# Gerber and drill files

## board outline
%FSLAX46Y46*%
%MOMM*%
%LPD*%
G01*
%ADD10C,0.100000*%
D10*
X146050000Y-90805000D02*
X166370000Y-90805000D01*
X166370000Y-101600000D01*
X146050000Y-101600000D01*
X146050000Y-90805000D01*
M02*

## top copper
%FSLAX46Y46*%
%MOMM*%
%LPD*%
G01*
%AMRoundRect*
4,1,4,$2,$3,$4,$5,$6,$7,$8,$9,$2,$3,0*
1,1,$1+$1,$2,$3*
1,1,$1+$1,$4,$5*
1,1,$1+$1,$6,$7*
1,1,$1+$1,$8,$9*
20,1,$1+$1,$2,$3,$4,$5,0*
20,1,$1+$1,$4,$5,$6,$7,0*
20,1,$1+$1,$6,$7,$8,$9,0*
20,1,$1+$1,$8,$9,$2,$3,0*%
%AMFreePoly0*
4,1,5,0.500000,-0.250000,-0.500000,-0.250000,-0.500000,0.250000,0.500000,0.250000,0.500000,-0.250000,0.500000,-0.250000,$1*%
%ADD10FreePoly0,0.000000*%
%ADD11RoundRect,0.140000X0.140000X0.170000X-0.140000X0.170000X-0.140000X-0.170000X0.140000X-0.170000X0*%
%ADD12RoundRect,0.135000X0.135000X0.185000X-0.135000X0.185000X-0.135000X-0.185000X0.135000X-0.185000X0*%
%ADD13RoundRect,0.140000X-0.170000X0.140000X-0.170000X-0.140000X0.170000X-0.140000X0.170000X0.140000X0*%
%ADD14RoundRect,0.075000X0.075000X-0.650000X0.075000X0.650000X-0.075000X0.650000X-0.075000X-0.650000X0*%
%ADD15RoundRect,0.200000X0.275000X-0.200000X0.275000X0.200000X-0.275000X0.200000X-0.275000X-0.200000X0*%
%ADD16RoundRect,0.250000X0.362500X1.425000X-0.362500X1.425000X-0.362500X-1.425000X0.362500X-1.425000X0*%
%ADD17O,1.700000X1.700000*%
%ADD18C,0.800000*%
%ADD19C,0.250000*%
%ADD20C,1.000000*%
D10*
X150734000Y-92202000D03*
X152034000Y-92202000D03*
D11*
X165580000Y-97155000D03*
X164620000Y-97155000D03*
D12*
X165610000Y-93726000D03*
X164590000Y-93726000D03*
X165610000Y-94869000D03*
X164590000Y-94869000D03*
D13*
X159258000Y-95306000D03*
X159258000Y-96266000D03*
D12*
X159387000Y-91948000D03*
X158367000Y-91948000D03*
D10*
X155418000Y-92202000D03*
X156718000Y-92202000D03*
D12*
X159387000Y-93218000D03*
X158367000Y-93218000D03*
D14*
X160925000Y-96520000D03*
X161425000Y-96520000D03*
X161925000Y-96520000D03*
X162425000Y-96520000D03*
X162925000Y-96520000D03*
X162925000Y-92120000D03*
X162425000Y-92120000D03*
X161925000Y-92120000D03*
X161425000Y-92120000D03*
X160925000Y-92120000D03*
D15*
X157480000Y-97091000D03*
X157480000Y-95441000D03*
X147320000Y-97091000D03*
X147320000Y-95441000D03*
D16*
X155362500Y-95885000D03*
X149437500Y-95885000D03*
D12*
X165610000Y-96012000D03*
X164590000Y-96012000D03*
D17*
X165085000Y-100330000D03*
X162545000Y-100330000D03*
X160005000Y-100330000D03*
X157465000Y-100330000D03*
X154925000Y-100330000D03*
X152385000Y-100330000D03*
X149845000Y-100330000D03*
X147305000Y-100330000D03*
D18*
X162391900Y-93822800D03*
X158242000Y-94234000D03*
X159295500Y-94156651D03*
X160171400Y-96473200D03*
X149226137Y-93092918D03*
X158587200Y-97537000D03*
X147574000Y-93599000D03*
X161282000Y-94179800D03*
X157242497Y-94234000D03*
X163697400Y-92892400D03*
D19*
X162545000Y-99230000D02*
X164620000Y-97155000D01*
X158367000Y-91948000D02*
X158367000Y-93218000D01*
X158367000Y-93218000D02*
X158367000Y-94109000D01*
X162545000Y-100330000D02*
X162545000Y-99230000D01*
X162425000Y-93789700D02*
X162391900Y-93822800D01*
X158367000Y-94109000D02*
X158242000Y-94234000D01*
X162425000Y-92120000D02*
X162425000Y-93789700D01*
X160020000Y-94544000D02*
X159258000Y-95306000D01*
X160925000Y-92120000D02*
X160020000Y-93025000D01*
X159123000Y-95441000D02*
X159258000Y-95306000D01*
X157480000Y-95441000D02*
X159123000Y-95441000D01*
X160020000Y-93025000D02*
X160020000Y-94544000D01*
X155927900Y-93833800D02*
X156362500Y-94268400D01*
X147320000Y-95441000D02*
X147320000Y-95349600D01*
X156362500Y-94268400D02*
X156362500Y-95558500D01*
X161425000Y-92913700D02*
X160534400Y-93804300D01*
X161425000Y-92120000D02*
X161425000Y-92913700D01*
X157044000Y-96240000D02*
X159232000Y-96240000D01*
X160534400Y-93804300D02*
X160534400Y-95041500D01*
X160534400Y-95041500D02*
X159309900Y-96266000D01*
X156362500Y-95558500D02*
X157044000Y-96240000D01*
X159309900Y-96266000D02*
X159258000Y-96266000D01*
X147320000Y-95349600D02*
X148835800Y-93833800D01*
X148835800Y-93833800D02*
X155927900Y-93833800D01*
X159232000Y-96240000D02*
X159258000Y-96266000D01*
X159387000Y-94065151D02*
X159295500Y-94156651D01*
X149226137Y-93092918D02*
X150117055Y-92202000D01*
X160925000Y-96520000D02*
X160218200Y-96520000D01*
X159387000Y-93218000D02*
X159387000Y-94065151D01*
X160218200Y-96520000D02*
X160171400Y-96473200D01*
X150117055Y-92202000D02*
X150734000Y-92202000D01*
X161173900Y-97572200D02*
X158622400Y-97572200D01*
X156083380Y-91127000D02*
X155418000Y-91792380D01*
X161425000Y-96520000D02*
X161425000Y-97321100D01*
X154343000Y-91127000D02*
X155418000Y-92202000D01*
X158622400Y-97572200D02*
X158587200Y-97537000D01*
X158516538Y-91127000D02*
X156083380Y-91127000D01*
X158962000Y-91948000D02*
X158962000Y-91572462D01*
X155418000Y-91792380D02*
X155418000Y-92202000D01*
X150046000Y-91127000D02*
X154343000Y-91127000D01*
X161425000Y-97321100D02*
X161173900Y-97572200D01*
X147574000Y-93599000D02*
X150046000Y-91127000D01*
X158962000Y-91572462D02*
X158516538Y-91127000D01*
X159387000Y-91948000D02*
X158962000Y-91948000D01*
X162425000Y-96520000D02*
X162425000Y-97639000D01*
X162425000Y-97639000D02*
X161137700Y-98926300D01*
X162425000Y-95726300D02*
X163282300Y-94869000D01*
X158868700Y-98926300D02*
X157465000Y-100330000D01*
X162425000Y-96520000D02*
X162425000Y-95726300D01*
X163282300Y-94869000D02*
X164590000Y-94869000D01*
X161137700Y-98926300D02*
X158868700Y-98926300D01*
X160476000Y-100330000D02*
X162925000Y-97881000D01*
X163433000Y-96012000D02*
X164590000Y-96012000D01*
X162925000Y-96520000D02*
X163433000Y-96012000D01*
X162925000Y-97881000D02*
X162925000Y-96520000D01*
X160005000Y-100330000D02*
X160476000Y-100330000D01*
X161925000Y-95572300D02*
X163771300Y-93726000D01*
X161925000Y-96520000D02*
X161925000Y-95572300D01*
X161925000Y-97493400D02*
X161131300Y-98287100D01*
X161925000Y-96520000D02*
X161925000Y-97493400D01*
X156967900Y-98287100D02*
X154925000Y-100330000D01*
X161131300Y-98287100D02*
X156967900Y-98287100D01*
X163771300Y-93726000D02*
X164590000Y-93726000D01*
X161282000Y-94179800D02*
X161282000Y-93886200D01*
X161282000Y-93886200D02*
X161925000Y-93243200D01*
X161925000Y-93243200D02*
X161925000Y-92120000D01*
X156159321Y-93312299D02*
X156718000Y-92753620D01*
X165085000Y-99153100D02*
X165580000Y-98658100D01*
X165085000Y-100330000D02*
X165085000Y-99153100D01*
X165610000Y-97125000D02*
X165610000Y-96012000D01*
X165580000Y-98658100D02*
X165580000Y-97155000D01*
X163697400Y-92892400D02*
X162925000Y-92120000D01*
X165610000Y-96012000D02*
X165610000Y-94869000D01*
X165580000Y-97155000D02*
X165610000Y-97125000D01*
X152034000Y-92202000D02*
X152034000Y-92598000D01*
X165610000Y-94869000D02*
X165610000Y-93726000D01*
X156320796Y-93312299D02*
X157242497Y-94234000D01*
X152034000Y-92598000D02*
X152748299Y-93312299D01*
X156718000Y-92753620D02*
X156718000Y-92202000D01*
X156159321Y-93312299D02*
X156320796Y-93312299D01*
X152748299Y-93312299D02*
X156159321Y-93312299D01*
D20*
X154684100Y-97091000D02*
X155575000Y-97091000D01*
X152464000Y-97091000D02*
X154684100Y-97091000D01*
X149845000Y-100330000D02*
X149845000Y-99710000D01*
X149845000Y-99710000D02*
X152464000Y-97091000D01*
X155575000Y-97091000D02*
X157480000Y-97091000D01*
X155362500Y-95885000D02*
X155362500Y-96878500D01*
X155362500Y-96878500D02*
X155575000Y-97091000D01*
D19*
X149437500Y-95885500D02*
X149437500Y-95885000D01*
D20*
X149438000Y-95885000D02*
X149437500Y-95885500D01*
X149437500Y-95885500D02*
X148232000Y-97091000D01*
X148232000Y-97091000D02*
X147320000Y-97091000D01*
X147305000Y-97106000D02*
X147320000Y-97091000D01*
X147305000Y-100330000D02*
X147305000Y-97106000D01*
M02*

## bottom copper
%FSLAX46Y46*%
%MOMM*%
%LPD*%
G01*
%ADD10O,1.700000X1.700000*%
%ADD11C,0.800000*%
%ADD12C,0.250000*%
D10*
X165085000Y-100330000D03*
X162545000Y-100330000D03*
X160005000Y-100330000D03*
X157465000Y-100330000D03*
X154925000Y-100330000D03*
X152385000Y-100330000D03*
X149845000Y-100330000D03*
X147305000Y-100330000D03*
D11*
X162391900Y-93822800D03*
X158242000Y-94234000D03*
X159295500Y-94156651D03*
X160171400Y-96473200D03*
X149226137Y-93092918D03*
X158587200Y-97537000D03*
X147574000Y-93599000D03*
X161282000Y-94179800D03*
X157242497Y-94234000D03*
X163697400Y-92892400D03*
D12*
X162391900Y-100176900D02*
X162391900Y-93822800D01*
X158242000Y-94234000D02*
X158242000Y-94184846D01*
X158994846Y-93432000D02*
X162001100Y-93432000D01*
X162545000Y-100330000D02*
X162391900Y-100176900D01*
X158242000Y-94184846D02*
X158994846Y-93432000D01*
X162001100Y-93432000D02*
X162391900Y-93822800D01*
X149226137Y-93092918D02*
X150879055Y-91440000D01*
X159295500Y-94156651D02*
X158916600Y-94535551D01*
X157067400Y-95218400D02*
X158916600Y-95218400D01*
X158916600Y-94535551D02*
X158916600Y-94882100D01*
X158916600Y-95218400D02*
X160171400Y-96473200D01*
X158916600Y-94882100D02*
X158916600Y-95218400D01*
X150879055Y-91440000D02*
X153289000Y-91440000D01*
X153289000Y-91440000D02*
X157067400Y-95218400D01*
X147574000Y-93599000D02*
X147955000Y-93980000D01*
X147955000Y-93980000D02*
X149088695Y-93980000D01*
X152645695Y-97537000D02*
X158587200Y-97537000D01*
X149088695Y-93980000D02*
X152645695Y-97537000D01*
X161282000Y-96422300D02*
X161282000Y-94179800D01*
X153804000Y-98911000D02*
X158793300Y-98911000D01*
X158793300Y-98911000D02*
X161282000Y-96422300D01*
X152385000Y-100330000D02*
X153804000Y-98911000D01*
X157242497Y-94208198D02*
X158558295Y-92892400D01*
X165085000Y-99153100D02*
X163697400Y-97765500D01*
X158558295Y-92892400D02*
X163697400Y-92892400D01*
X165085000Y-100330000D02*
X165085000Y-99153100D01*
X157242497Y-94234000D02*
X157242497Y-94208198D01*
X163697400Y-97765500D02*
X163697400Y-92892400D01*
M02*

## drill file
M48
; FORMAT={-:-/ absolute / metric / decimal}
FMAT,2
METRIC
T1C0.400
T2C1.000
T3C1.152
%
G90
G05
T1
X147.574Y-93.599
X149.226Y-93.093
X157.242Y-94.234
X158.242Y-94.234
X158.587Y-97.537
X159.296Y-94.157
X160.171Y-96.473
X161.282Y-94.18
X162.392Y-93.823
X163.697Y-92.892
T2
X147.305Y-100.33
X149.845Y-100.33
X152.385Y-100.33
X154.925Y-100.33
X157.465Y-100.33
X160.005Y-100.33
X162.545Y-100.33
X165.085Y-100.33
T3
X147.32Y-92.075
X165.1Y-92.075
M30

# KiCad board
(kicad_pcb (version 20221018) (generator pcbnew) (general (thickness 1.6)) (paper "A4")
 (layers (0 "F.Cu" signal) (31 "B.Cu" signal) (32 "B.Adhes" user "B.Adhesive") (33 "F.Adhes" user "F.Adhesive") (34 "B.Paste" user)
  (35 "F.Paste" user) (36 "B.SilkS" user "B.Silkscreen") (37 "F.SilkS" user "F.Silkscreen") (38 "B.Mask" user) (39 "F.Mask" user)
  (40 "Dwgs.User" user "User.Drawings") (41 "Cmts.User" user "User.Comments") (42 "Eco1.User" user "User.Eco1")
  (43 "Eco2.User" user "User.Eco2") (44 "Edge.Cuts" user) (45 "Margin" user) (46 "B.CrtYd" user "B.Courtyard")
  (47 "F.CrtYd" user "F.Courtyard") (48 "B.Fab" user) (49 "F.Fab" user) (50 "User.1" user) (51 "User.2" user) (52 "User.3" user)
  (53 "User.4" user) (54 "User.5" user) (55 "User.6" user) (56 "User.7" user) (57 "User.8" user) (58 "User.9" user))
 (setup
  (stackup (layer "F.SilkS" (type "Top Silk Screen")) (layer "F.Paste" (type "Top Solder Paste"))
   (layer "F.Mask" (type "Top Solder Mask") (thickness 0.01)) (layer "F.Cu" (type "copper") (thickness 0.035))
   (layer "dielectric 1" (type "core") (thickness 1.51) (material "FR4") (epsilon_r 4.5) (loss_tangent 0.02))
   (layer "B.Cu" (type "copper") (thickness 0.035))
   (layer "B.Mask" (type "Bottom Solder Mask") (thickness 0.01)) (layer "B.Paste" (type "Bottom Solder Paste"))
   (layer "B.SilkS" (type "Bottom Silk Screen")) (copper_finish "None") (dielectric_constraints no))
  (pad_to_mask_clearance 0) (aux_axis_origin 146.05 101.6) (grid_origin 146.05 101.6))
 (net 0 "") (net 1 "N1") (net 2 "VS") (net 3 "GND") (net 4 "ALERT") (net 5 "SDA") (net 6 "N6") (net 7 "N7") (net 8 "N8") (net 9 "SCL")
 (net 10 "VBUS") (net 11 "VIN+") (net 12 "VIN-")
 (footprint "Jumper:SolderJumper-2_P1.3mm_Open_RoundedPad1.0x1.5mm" (layer "F.Cu") (at 151.384 92.202)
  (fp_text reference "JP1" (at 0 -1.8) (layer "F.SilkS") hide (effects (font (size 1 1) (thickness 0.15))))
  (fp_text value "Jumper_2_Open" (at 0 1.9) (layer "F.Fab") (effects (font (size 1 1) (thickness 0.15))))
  (pad "1" smd custom (at -0.65 0) (size 1 0.5) (layers "F.Cu" "F.Mask") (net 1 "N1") (zone_connect 2) (thermal_bridge_angle 45)
   (options (clearance outline) (anchor rect)) (primitives))
  (pad "2" smd custom (at 0.65 0) (size 1 0.5) (layers "F.Cu" "F.Mask") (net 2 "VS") (zone_connect 2) (thermal_bridge_angle 45)
   (options (clearance outline) (anchor rect)) (primitives)))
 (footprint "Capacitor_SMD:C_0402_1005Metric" (layer "F.Cu") (at 165.1 97.155 180)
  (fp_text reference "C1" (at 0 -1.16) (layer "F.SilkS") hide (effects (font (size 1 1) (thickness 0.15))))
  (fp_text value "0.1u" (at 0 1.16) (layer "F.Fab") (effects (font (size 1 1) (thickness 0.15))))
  (pad "1" smd roundrect (at -0.48 0 180) (size 0.56 0.62) (layers "F.Cu" "F.Paste" "F.Mask") (roundrect_rratio 0.25) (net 2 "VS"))
  (pad "2" smd roundrect (at 0.48 0 180) (size 0.56 0.62) (layers "F.Cu" "F.Paste" "F.Mask") (roundrect_rratio 0.25) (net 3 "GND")))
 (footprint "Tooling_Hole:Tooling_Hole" (layer "F.Cu") (at 165.1 92.075)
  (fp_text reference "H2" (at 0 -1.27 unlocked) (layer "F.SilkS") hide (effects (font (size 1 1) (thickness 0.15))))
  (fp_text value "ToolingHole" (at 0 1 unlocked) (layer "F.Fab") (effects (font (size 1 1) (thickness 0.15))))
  (pad "" np_thru_hole circle (at 0 0) (size 1.152 1.152) (drill 1.152) (layers "F&B.Cu" "*.Mask")))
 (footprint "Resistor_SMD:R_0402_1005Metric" (layer "F.Cu") (at 165.1 93.726 180)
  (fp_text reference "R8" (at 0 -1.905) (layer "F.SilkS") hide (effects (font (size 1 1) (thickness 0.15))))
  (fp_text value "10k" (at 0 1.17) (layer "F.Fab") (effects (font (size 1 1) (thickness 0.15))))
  (pad "1" smd roundrect (at -0.51 0 180) (size 0.54 0.64) (layers "F.Cu" "F.Paste" "F.Mask") (roundrect_rratio 0.25) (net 2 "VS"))
  (pad "2" smd roundrect (at 0.51 0 180) (size 0.54 0.64) (layers "F.Cu" "F.Paste" "F.Mask") (roundrect_rratio 0.25) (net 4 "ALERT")))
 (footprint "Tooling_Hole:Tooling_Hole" (layer "F.Cu") (at 147.32 92.075)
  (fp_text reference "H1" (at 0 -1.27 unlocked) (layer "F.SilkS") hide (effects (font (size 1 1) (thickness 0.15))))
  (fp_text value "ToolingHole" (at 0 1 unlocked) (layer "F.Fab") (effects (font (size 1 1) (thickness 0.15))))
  (pad "" np_thru_hole circle (at 0 0) (size 1.152 1.152) (drill 1.152) (layers "F&B.Cu" "*.Mask")))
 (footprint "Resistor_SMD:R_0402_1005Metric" (layer "F.Cu") (at 165.1 94.869 180)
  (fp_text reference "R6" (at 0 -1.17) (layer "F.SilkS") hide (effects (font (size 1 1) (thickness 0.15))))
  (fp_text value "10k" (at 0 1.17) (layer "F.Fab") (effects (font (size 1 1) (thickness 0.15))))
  (pad "1" smd roundrect (at -0.51 0 180) (size 0.54 0.64) (layers "F.Cu" "F.Paste" "F.Mask") (roundrect_rratio 0.25) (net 2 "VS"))
  (pad "2" smd roundrect (at 0.51 0 180) (size 0.54 0.64) (layers "F.Cu" "F.Paste" "F.Mask") (roundrect_rratio 0.25) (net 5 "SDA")))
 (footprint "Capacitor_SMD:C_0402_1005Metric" (layer "F.Cu") (at 159.258 95.786 -90)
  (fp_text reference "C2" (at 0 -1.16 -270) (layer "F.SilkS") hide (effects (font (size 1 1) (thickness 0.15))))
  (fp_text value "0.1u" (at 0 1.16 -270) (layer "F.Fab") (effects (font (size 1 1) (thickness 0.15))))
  (pad "1" smd roundrect (at -0.48 0 270) (size 0.56 0.62) (layers "F.Cu" "F.Paste" "F.Mask") (roundrect_rratio 0.25) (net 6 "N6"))
  (pad "2" smd roundrect (at 0.48 0 270) (size 0.56 0.62) (layers "F.Cu" "F.Paste" "F.Mask") (roundrect_rratio 0.25) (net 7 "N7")))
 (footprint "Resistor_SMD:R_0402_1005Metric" (layer "F.Cu") (at 158.877 91.948 180)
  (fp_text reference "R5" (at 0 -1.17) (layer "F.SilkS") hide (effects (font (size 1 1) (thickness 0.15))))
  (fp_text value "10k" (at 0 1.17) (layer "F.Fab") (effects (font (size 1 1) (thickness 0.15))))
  (pad "1" smd roundrect (at -0.51 0 180) (size 0.54 0.64) (layers "F.Cu" "F.Paste" "F.Mask") (roundrect_rratio 0.25) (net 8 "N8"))
  (pad "2" smd roundrect (at 0.51 0 180) (size 0.54 0.64) (layers "F.Cu" "F.Paste" "F.Mask") (roundrect_rratio 0.25) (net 3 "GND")))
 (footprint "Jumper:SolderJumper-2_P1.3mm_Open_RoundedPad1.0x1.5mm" (layer "F.Cu") (at 156.068 92.202)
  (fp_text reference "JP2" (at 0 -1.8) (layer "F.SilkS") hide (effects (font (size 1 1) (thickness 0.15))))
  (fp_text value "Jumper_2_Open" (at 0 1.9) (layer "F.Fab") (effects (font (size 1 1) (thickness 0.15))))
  (pad "1" smd custom (at -0.65 0) (size 1 0.5) (layers "F.Cu" "F.Mask") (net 8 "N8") (zone_connect 2) (thermal_bridge_angle 45)
   (options (clearance outline) (anchor rect)) (primitives))
  (pad "2" smd custom (at 0.65 0) (size 1 0.5) (layers "F.Cu" "F.Mask") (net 2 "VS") (zone_connect 2) (thermal_bridge_angle 45)
   (options (clearance outline) (anchor rect)) (primitives)))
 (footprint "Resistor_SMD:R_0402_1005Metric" (layer "F.Cu") (at 158.877 93.218 180)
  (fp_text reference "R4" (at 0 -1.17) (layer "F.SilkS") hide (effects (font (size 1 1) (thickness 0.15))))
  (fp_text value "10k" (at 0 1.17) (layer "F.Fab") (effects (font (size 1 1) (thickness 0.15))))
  (pad "1" smd roundrect (at -0.51 0 180) (size 0.54 0.64) (layers "F.Cu" "F.Paste" "F.Mask") (roundrect_rratio 0.25) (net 1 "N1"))
  (pad "2" smd roundrect (at 0.51 0 180) (size 0.54 0.64) (layers "F.Cu" "F.Paste" "F.Mask") (roundrect_rratio 0.25) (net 3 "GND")))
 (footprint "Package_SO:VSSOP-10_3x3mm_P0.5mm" (layer "F.Cu") (at 161.925 94.32 90)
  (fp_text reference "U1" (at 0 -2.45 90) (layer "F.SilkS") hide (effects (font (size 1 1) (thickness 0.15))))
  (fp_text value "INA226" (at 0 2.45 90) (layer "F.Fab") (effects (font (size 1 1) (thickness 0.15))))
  (pad "1" smd roundrect (at -2.2 -1 90) (size 1.45 0.3) (layers "F.Cu" "F.Paste" "F.Mask") (roundrect_rratio 0.25) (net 1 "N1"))
  (pad "2" smd roundrect (at -2.2 -0.5 90) (size 1.45 0.3) (layers "F.Cu" "F.Paste" "F.Mask") (roundrect_rratio 0.25) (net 8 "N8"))
  (pad "3" smd roundrect (at -2.2 0 90) (size 1.45 0.3) (layers "F.Cu" "F.Paste" "F.Mask") (roundrect_rratio 0.25) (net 4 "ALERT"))
  (pad "4" smd roundrect (at -2.2 0.5 90) (size 1.45 0.3) (layers "F.Cu" "F.Paste" "F.Mask") (roundrect_rratio 0.25) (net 5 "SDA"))
  (pad "5" smd roundrect (at -2.2 1 90) (size 1.45 0.3) (layers "F.Cu" "F.Paste" "F.Mask") (roundrect_rratio 0.25) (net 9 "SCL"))
  (pad "6" smd roundrect (at 2.2 1 90) (size 1.45 0.3) (layers "F.Cu" "F.Paste" "F.Mask") (roundrect_rratio 0.25) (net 2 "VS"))
  (pad "7" smd roundrect (at 2.2 0.5 90) (size 1.45 0.3) (layers "F.Cu" "F.Paste" "F.Mask") (roundrect_rratio 0.25) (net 3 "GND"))
  (pad "8" smd roundrect (at 2.2 0 90) (size 1.45 0.3) (layers "F.Cu" "F.Paste" "F.Mask") (roundrect_rratio 0.25) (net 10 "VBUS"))
  (pad "9" smd roundrect (at 2.2 -0.5 90) (size 1.45 0.3) (layers "F.Cu" "F.Paste" "F.Mask") (roundrect_rratio 0.25) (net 7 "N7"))
  (pad "10" smd roundrect (at 2.2 -1 90) (size 1.45 0.3) (layers "F.Cu" "F.Paste" "F.Mask") (roundrect_rratio 0.25) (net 6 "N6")))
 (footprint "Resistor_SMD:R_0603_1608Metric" (layer "F.Cu") (at 157.48 96.266 90)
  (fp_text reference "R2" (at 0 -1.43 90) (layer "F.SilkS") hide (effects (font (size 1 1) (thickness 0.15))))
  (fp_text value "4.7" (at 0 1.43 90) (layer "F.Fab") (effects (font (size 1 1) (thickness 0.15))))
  (pad "1" smd roundrect (at -0.825 0 90) (size 0.8 0.95) (layers "F.Cu" "F.Paste" "F.Mask") (roundrect_rratio 0.25) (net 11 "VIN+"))
  (pad "2" smd roundrect (at 0.825 0 90) (size 0.8 0.95) (layers "F.Cu" "F.Paste" "F.Mask") (roundrect_rratio 0.25) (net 6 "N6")))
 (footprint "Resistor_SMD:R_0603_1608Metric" (layer "F.Cu") (at 147.32 96.266 90)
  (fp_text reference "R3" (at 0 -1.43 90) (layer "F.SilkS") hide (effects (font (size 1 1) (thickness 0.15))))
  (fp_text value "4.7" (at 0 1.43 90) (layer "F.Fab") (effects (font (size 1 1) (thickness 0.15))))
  (pad "1" smd roundrect (at -0.825 0 90) (size 0.8 0.95) (layers "F.Cu" "F.Paste" "F.Mask") (roundrect_rratio 0.25) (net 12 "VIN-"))
  (pad "2" smd roundrect (at 0.825 0 90) (size 0.8 0.95) (layers "F.Cu" "F.Paste" "F.Mask") (roundrect_rratio 0.25) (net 7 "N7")))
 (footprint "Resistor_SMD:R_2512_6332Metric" (layer "F.Cu") (at 152.4 95.885 180)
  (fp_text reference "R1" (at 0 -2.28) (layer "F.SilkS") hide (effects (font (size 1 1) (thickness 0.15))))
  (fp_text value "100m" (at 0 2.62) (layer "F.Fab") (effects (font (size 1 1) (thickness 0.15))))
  (pad "1" smd roundrect (at -2.9625 0 180) (size 1.225 3.35) (layers "F.Cu" "F.Paste" "F.Mask") (roundrect_rratio 0.2040816327)
   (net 11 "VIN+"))
  (pad "2" smd roundrect (at 2.9625 0 180) (size 1.225 3.35) (layers "F.Cu" "F.Paste" "F.Mask") (roundrect_rratio 0.2040816327)
   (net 12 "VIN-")))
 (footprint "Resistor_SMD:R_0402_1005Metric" (layer "F.Cu") (at 165.1 96.012 180)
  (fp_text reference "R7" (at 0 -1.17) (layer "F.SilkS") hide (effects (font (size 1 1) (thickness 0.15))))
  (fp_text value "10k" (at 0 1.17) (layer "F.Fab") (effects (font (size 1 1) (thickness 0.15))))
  (pad "1" smd roundrect (at -0.51 0 180) (size 0.54 0.64) (layers "F.Cu" "F.Paste" "F.Mask") (roundrect_rratio 0.25) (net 2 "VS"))
  (pad "2" smd roundrect (at 0.51 0 180) (size 0.54 0.64) (layers "F.Cu" "F.Paste" "F.Mask") (roundrect_rratio 0.25) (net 9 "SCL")))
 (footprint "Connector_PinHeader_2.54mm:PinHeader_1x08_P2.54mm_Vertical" (layer "B.Cu") (at 165.085 100.33 90)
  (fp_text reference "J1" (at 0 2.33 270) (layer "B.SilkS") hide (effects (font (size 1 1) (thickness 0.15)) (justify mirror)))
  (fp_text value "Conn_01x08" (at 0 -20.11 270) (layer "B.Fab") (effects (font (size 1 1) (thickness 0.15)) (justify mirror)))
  (pad "1" thru_hole oval (at 0 0 90) (size 1.7 1.7) (drill 1) (layers "*.Cu" "*.Mask") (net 2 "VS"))
  (pad "2" thru_hole oval (at 0 -2.54 90) (size 1.7 1.7) (drill 1) (layers "*.Cu" "*.Mask") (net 3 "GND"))
  (pad "3" thru_hole oval (at 0 -5.08 90) (size 1.7 1.7) (drill 1) (layers "*.Cu" "*.Mask") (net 9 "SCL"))
  (pad "4" thru_hole oval (at 0 -7.62 90) (size 1.7 1.7) (drill 1) (layers "*.Cu" "*.Mask") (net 5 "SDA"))
  (pad "5" thru_hole oval (at 0 -10.16 90) (size 1.7 1.7) (drill 1) (layers "*.Cu" "*.Mask") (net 4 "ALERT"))
  (pad "6" thru_hole oval (at 0 -12.7 90) (size 1.7 1.7) (drill 1) (layers "*.Cu" "*.Mask") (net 10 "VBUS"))
  (pad "7" thru_hole oval (at 0 -15.24 90) (size 1.7 1.7) (drill 1) (layers "*.Cu" "*.Mask") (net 11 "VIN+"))
  (pad "8" thru_hole oval (at 0 -17.78 90) (size 1.7 1.7) (drill 1) (layers "*.Cu" "*.Mask") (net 12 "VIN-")))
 (gr_rect (start 146.05 90.805) (end 166.37 101.6) (stroke (width 0.1) (type default)) (fill none) (layer "Edge.Cuts"))
 (segment (start 162.545 99.23) (end 164.62 97.155) (width 0.25) (layer "F.Cu") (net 3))
 (segment (start 158.367 91.948) (end 158.367 93.218) (width 0.25) (layer "F.Cu") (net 3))
 (segment (start 158.367 93.218) (end 158.367 94.109) (width 0.25) (layer "F.Cu") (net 3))
 (segment (start 162.545 100.33) (end 162.545 99.23) (width 0.25) (layer "F.Cu") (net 3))
 (segment (start 162.425 93.7897) (end 162.3919 93.8228) (width 0.25) (layer "F.Cu") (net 3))
 (segment (start 158.367 94.109) (end 158.242 94.234) (width 0.25) (layer "F.Cu") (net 3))
 (segment (start 162.425 92.12) (end 162.425 93.7897) (width 0.25) (layer "F.Cu") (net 3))
 (via (at 162.3919 93.8228) (size 0.8) (drill 0.4) (layers "F.Cu" "B.Cu") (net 3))
 (via (at 158.242 94.234) (size 0.8) (drill 0.4) (layers "F.Cu" "B.Cu") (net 3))
 (segment (start 162.3919 100.1769) (end 162.3919 93.8228) (width 0.25) (layer "B.Cu") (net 3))
 (segment (start 158.242 94.234) (end 158.242 94.184846) (width 0.25) (layer "B.Cu") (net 3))
 (segment (start 158.994846 93.432) (end 162.0011 93.432) (width 0.25) (layer "B.Cu") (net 3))
 (segment (start 162.545 100.33) (end 162.3919 100.1769) (width 0.25) (layer "B.Cu") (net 3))
 (segment (start 158.242 94.184846) (end 158.994846 93.432) (width 0.25) (layer "B.Cu") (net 3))
 (segment (start 162.0011 93.432) (end 162.3919 93.8228) (width 0.25) (layer "B.Cu") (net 3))
 (segment (start 160.02 94.544) (end 159.258 95.306) (width 0.25) (layer "F.Cu") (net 6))
 (segment (start 160.925 92.12) (end 160.02 93.025) (width 0.25) (layer "F.Cu") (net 6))
 (segment (start 159.123 95.441) (end 159.258 95.306) (width 0.25) (layer "F.Cu") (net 6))
 (segment (start 157.48 95.441) (end 159.123 95.441) (width 0.25) (layer "F.Cu") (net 6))
 (segment (start 160.02 93.025) (end 160.02 94.544) (width 0.25) (layer "F.Cu") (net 6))
 (segment (start 155.9279 93.8338) (end 156.3625 94.2684) (width 0.25) (layer "F.Cu") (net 7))
 (segment (start 147.32 95.441) (end 147.32 95.3496) (width 0.25) (layer "F.Cu") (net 7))
 (segment (start 156.3625 94.2684) (end 156.3625 95.5585) (width 0.25) (layer "F.Cu") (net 7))
 (segment (start 161.425 92.9137) (end 160.5344 93.8043) (width 0.25) (layer "F.Cu") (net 7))
 (segment (start 161.425 92.12) (end 161.425 92.9137) (width 0.25) (layer "F.Cu") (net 7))
 (segment (start 157.044 96.24) (end 159.232 96.24) (width 0.25) (layer "F.Cu") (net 7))
 (segment (start 160.5344 93.8043) (end 160.5344 95.0415) (width 0.25) (layer "F.Cu") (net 7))
 (segment (start 160.5344 95.0415) (end 159.3099 96.266) (width 0.25) (layer "F.Cu") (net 7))
 (segment (start 156.3625 95.5585) (end 157.044 96.24) (width 0.25) (layer "F.Cu") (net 7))
 (segment (start 159.3099 96.266) (end 159.258 96.266) (width 0.25) (layer "F.Cu") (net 7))
 (segment (start 147.32 95.3496) (end 148.8358 93.8338) (width 0.25) (layer "F.Cu") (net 7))
 (segment (start 148.8358 93.8338) (end 155.9279 93.8338) (width 0.25) (layer "F.Cu") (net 7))
 (segment (start 159.232 96.24) (end 159.258 96.266) (width 0.25) (layer "F.Cu") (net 7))
 (segment (start 159.387 94.065151) (end 159.2955 94.156651) (width 0.25) (layer "F.Cu") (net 1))
 (segment (start 149.226137 93.092918) (end 150.117055 92.202) (width 0.25) (layer "F.Cu") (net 1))
 (segment (start 160.925 96.52) (end 160.2182 96.52) (width 0.25) (layer "F.Cu") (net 1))
 (segment (start 159.387 93.218) (end 159.387 94.065151) (width 0.25) (layer "F.Cu") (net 1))
 (segment (start 160.2182 96.52) (end 160.1714 96.4732) (width 0.25) (layer "F.Cu") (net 1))
 (segment (start 150.117055 92.202) (end 150.734 92.202) (width 0.25) (layer "F.Cu") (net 1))
 (via (at 159.2955 94.156651) (size 0.8) (drill 0.4) (layers "F.Cu" "B.Cu") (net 1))
 (via (at 160.1714 96.4732) (size 0.8) (drill 0.4) (layers "F.Cu" "B.Cu") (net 1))
 (via (at 149.226137 93.092918) (size 0.8) (drill 0.4) (layers "F.Cu" "B.Cu") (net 1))
 (segment (start 149.226137 93.092918) (end 150.879055 91.44) (width 0.25) (layer "B.Cu") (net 1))
 (segment (start 159.2955 94.156651) (end 158.9166 94.535551) (width 0.25) (layer "B.Cu") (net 1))
 (segment (start 157.0674 95.2184) (end 158.9166 95.2184) (width 0.25) (layer "B.Cu") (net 1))
 (segment (start 158.9166 94.535551) (end 158.9166 94.8821) (width 0.25) (layer "B.Cu") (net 1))
 (segment (start 158.9166 95.2184) (end 160.1714 96.4732) (width 0.25) (layer "B.Cu") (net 1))
 (segment (start 158.9166 94.8821) (end 158.9166 95.2184) (width 0.25) (layer "B.Cu") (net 1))
 (segment (start 150.879055 91.44) (end 153.289 91.44) (width 0.25) (layer "B.Cu") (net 1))
 (segment (start 153.289 91.44) (end 157.0674 95.2184) (width 0.25) (layer "B.Cu") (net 1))
 (segment (start 161.1739 97.5722) (end 158.6224 97.5722) (width 0.25) (layer "F.Cu") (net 8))
 (segment (start 156.08338 91.127) (end 155.418 91.79238) (width 0.25) (layer "F.Cu") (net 8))
 (segment (start 161.425 96.52) (end 161.425 97.3211) (width 0.25) (layer "F.Cu") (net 8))
 (segment (start 154.343 91.127) (end 155.418 92.202) (width 0.25) (layer "F.Cu") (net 8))
 (segment (start 158.6224 97.5722) (end 158.5872 97.537) (width 0.25) (layer "F.Cu") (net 8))
 (segment (start 158.516538 91.127) (end 156.08338 91.127) (width 0.25) (layer "F.Cu") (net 8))
 (segment (start 158.962 91.948) (end 158.962 91.572462) (width 0.25) (layer "F.Cu") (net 8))
 (segment (start 155.418 91.79238) (end 155.418 92.202) (width 0.25) (layer "F.Cu") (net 8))
 (segment (start 150.046 91.127) (end 154.343 91.127) (width 0.25) (layer "F.Cu") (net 8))
 (segment (start 161.425 97.3211) (end 161.1739 97.5722) (width 0.25) (layer "F.Cu") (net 8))
 (segment (start 147.574 93.599) (end 150.046 91.127) (width 0.25) (layer "F.Cu") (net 8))
 (segment (start 158.962 91.572462) (end 158.516538 91.127) (width 0.25) (layer "F.Cu") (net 8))
 (segment (start 159.387 91.948) (end 158.962 91.948) (width 0.25) (layer "F.Cu") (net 8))
 (via (at 158.5872 97.537) (size 0.8) (drill 0.4) (layers "F.Cu" "B.Cu") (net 8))
 (via (at 147.574 93.599) (size 0.8) (drill 0.4) (layers "F.Cu" "B.Cu") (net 8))
 (segment (start 147.574 93.599) (end 147.955 93.98) (width 0.25) (layer "B.Cu") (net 8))
 (segment (start 147.955 93.98) (end 149.088695 93.98) (width 0.25) (layer "B.Cu") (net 8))
 (segment (start 152.645695 97.537) (end 158.5872 97.537) (width 0.25) (layer "B.Cu") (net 8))
 (segment (start 149.088695 93.98) (end 152.645695 97.537) (width 0.25) (layer "B.Cu") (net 8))
 (segment (start 162.425 96.52) (end 162.425 97.639) (width 0.25) (layer "F.Cu") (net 5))
 (segment (start 162.425 97.639) (end 161.1377 98.9263) (width 0.25) (layer "F.Cu") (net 5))
 (segment (start 162.425 95.7263) (end 163.2823 94.869) (width 0.25) (layer "F.Cu") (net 5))
 (segment (start 158.8687 98.9263) (end 157.465 100.33) (width 0.25) (layer "F.Cu") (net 5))
 (segment (start 162.425 96.52) (end 162.425 95.7263) (width 0.25) (layer "F.Cu") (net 5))
 (segment (start 163.2823 94.869) (end 164.59 94.869) (width 0.25) (layer "F.Cu") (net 5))
 (segment (start 161.1377 98.9263) (end 158.8687 98.9263) (width 0.25) (layer "F.Cu") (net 5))
 (segment (start 160.476 100.33) (end 162.925 97.881) (width 0.25) (layer "F.Cu") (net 9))
 (segment (start 163.433 96.012) (end 164.59 96.012) (width 0.25) (layer "F.Cu") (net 9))
 (segment (start 162.925 96.52) (end 163.433 96.012) (width 0.25) (layer "F.Cu") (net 9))
 (segment (start 162.925 97.881) (end 162.925 96.52) (width 0.25) (layer "F.Cu") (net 9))
 (segment (start 160.005 100.33) (end 160.476 100.33) (width 0.25) (layer "F.Cu") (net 9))
 (segment (start 161.925 95.5723) (end 163.7713 93.726) (width 0.25) (layer "F.Cu") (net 4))
 (segment (start 161.925 96.52) (end 161.925 95.5723) (width 0.25) (layer "F.Cu") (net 4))
 (segment (start 161.925 97.4934) (end 161.1313 98.2871) (width 0.25) (layer "F.Cu") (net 4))
 (segment (start 161.925 96.52) (end 161.925 97.4934) (width 0.25) (layer "F.Cu") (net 4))
 (segment (start 156.9679 98.2871) (end 154.925 100.33) (width 0.25) (layer "F.Cu") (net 4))
 (segment (start 161.1313 98.2871) (end 156.9679 98.2871) (width 0.25) (layer "F.Cu") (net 4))
 (segment (start 163.7713 93.726) (end 164.59 93.726) (width 0.25) (layer "F.Cu") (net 4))
 (segment (start 161.282 94.1798) (end 161.282 93.8862) (width 0.25) (layer "F.Cu") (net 10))
 (segment (start 161.282 93.8862) (end 161.925 93.2432) (width 0.25) (layer "F.Cu") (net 10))
 (segment (start 161.925 93.2432) (end 161.925 92.12) (width 0.25) (layer "F.Cu") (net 10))
 (via (at 161.282 94.1798) (size 0.8) (drill 0.4) (layers "F.Cu" "B.Cu") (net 10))
 (segment (start 161.282 96.4223) (end 161.282 94.1798) (width 0.25) (layer "B.Cu") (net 10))
 (segment (start 153.804 98.911) (end 158.7933 98.911) (width 0.25) (layer "B.Cu") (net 10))
 (segment (start 158.7933 98.911) (end 161.282 96.4223) (width 0.25) (layer "B.Cu") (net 10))
 (segment (start 152.385 100.33) (end 153.804 98.911) (width 0.25) (layer "B.Cu") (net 10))
 (segment (start 156.159321 93.312299) (end 156.718 92.75362) (width 0.25) (layer "F.Cu") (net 2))
 (segment (start 165.085 99.1531) (end 165.58 98.6581) (width 0.25) (layer "F.Cu") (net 2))
 (segment (start 165.085 100.33) (end 165.085 99.1531) (width 0.25) (layer "F.Cu") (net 2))
 (segment (start 165.61 97.125) (end 165.61 96.012) (width 0.25) (layer "F.Cu") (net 2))
 (segment (start 165.58 98.6581) (end 165.58 97.155) (width 0.25) (layer "F.Cu") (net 2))
 (segment (start 163.6974 92.8924) (end 162.925 92.12) (width 0.25) (layer "F.Cu") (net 2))
 (segment (start 165.61 96.012) (end 165.61 94.869) (width 0.25) (layer "F.Cu") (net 2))
 (segment (start 165.58 97.155) (end 165.61 97.125) (width 0.25) (layer "F.Cu") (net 2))
 (segment (start 152.034 92.202) (end 152.034 92.598) (width 0.25) (layer "F.Cu") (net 2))
 (segment (start 165.61 94.869) (end 165.61 93.726) (width 0.25) (layer "F.Cu") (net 2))
 (segment (start 156.320796 93.312299) (end 157.242497 94.234) (width 0.25) (layer "F.Cu") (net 2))
 (segment (start 152.034 92.598) (end 152.748299 93.312299) (width 0.25) (layer "F.Cu") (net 2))
 (segment (start 156.718 92.75362) (end 156.718 92.202) (width 0.25) (layer "F.Cu") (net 2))
 (segment (start 156.159321 93.312299) (end 156.320796 93.312299) (width 0.25) (layer "F.Cu") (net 2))
 (segment (start 152.748299 93.312299) (end 156.159321 93.312299) (width 0.25) (layer "F.Cu") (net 2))
 (via (at 157.242497 94.234) (size 0.8) (drill 0.4) (layers "F.Cu" "B.Cu") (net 2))
 (via (at 163.6974 92.8924) (size 0.8) (drill 0.4) (layers "F.Cu" "B.Cu") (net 2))
 (segment (start 157.242497 94.208198) (end 158.558295 92.8924) (width 0.25) (layer "B.Cu") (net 2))
 (segment (start 165.085 99.1531) (end 163.6974 97.7655) (width 0.25) (layer "B.Cu") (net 2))
 (segment (start 158.558295 92.8924) (end 163.6974 92.8924) (width 0.25) (layer "B.Cu") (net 2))
 (segment (start 165.085 100.33) (end 165.085 99.1531) (width 0.25) (layer "B.Cu") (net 2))
 (segment (start 157.242497 94.234) (end 157.242497 94.208198) (width 0.25) (layer "B.Cu") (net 2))
 (segment (start 163.6974 97.7655) (end 163.6974 92.8924) (width 0.25) (layer "B.Cu") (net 2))
 (segment (start 154.6841 97.091) (end 155.575 97.091) (width 1) (layer "F.Cu") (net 11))
 (segment (start 152.464 97.091) (end 154.6841 97.091) (width 1) (layer "F.Cu") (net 11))
 (segment (start 149.845 100.33) (end 149.845 99.71) (width 1) (layer "F.Cu") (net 11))
 (segment (start 149.845 99.71) (end 152.464 97.091) (width 1) (layer "F.Cu") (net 11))
 (segment (start 155.575 97.091) (end 157.48 97.091) (width 1) (layer "F.Cu") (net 11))
 (segment (start 155.3625 95.885) (end 155.3625 96.8785) (width 1) (layer "F.Cu") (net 11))
 (segment (start 155.3625 96.8785) (end 155.575 97.091) (width 1) (layer "F.Cu") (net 11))
 (segment (start 149.4375 95.8855) (end 149.4375 95.885) (width 0.25) (layer "F.Cu") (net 12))
 (segment (start 149.438 95.885) (end 149.4375 95.8855) (width 1) (layer "F.Cu") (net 12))
 (segment (start 149.4375 95.8855) (end 148.232 97.091) (width 1) (layer "F.Cu") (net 12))
 (segment (start 148.232 97.091) (end 147.32 97.091) (width 1) (layer "F.Cu") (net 12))
 (segment (start 147.305 97.106) (end 147.32 97.091) (width 1) (layer "F.Cu") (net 12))
 (segment (start 147.305 100.33) (end 147.305 97.106) (width 1) (layer "F.Cu") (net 12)))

